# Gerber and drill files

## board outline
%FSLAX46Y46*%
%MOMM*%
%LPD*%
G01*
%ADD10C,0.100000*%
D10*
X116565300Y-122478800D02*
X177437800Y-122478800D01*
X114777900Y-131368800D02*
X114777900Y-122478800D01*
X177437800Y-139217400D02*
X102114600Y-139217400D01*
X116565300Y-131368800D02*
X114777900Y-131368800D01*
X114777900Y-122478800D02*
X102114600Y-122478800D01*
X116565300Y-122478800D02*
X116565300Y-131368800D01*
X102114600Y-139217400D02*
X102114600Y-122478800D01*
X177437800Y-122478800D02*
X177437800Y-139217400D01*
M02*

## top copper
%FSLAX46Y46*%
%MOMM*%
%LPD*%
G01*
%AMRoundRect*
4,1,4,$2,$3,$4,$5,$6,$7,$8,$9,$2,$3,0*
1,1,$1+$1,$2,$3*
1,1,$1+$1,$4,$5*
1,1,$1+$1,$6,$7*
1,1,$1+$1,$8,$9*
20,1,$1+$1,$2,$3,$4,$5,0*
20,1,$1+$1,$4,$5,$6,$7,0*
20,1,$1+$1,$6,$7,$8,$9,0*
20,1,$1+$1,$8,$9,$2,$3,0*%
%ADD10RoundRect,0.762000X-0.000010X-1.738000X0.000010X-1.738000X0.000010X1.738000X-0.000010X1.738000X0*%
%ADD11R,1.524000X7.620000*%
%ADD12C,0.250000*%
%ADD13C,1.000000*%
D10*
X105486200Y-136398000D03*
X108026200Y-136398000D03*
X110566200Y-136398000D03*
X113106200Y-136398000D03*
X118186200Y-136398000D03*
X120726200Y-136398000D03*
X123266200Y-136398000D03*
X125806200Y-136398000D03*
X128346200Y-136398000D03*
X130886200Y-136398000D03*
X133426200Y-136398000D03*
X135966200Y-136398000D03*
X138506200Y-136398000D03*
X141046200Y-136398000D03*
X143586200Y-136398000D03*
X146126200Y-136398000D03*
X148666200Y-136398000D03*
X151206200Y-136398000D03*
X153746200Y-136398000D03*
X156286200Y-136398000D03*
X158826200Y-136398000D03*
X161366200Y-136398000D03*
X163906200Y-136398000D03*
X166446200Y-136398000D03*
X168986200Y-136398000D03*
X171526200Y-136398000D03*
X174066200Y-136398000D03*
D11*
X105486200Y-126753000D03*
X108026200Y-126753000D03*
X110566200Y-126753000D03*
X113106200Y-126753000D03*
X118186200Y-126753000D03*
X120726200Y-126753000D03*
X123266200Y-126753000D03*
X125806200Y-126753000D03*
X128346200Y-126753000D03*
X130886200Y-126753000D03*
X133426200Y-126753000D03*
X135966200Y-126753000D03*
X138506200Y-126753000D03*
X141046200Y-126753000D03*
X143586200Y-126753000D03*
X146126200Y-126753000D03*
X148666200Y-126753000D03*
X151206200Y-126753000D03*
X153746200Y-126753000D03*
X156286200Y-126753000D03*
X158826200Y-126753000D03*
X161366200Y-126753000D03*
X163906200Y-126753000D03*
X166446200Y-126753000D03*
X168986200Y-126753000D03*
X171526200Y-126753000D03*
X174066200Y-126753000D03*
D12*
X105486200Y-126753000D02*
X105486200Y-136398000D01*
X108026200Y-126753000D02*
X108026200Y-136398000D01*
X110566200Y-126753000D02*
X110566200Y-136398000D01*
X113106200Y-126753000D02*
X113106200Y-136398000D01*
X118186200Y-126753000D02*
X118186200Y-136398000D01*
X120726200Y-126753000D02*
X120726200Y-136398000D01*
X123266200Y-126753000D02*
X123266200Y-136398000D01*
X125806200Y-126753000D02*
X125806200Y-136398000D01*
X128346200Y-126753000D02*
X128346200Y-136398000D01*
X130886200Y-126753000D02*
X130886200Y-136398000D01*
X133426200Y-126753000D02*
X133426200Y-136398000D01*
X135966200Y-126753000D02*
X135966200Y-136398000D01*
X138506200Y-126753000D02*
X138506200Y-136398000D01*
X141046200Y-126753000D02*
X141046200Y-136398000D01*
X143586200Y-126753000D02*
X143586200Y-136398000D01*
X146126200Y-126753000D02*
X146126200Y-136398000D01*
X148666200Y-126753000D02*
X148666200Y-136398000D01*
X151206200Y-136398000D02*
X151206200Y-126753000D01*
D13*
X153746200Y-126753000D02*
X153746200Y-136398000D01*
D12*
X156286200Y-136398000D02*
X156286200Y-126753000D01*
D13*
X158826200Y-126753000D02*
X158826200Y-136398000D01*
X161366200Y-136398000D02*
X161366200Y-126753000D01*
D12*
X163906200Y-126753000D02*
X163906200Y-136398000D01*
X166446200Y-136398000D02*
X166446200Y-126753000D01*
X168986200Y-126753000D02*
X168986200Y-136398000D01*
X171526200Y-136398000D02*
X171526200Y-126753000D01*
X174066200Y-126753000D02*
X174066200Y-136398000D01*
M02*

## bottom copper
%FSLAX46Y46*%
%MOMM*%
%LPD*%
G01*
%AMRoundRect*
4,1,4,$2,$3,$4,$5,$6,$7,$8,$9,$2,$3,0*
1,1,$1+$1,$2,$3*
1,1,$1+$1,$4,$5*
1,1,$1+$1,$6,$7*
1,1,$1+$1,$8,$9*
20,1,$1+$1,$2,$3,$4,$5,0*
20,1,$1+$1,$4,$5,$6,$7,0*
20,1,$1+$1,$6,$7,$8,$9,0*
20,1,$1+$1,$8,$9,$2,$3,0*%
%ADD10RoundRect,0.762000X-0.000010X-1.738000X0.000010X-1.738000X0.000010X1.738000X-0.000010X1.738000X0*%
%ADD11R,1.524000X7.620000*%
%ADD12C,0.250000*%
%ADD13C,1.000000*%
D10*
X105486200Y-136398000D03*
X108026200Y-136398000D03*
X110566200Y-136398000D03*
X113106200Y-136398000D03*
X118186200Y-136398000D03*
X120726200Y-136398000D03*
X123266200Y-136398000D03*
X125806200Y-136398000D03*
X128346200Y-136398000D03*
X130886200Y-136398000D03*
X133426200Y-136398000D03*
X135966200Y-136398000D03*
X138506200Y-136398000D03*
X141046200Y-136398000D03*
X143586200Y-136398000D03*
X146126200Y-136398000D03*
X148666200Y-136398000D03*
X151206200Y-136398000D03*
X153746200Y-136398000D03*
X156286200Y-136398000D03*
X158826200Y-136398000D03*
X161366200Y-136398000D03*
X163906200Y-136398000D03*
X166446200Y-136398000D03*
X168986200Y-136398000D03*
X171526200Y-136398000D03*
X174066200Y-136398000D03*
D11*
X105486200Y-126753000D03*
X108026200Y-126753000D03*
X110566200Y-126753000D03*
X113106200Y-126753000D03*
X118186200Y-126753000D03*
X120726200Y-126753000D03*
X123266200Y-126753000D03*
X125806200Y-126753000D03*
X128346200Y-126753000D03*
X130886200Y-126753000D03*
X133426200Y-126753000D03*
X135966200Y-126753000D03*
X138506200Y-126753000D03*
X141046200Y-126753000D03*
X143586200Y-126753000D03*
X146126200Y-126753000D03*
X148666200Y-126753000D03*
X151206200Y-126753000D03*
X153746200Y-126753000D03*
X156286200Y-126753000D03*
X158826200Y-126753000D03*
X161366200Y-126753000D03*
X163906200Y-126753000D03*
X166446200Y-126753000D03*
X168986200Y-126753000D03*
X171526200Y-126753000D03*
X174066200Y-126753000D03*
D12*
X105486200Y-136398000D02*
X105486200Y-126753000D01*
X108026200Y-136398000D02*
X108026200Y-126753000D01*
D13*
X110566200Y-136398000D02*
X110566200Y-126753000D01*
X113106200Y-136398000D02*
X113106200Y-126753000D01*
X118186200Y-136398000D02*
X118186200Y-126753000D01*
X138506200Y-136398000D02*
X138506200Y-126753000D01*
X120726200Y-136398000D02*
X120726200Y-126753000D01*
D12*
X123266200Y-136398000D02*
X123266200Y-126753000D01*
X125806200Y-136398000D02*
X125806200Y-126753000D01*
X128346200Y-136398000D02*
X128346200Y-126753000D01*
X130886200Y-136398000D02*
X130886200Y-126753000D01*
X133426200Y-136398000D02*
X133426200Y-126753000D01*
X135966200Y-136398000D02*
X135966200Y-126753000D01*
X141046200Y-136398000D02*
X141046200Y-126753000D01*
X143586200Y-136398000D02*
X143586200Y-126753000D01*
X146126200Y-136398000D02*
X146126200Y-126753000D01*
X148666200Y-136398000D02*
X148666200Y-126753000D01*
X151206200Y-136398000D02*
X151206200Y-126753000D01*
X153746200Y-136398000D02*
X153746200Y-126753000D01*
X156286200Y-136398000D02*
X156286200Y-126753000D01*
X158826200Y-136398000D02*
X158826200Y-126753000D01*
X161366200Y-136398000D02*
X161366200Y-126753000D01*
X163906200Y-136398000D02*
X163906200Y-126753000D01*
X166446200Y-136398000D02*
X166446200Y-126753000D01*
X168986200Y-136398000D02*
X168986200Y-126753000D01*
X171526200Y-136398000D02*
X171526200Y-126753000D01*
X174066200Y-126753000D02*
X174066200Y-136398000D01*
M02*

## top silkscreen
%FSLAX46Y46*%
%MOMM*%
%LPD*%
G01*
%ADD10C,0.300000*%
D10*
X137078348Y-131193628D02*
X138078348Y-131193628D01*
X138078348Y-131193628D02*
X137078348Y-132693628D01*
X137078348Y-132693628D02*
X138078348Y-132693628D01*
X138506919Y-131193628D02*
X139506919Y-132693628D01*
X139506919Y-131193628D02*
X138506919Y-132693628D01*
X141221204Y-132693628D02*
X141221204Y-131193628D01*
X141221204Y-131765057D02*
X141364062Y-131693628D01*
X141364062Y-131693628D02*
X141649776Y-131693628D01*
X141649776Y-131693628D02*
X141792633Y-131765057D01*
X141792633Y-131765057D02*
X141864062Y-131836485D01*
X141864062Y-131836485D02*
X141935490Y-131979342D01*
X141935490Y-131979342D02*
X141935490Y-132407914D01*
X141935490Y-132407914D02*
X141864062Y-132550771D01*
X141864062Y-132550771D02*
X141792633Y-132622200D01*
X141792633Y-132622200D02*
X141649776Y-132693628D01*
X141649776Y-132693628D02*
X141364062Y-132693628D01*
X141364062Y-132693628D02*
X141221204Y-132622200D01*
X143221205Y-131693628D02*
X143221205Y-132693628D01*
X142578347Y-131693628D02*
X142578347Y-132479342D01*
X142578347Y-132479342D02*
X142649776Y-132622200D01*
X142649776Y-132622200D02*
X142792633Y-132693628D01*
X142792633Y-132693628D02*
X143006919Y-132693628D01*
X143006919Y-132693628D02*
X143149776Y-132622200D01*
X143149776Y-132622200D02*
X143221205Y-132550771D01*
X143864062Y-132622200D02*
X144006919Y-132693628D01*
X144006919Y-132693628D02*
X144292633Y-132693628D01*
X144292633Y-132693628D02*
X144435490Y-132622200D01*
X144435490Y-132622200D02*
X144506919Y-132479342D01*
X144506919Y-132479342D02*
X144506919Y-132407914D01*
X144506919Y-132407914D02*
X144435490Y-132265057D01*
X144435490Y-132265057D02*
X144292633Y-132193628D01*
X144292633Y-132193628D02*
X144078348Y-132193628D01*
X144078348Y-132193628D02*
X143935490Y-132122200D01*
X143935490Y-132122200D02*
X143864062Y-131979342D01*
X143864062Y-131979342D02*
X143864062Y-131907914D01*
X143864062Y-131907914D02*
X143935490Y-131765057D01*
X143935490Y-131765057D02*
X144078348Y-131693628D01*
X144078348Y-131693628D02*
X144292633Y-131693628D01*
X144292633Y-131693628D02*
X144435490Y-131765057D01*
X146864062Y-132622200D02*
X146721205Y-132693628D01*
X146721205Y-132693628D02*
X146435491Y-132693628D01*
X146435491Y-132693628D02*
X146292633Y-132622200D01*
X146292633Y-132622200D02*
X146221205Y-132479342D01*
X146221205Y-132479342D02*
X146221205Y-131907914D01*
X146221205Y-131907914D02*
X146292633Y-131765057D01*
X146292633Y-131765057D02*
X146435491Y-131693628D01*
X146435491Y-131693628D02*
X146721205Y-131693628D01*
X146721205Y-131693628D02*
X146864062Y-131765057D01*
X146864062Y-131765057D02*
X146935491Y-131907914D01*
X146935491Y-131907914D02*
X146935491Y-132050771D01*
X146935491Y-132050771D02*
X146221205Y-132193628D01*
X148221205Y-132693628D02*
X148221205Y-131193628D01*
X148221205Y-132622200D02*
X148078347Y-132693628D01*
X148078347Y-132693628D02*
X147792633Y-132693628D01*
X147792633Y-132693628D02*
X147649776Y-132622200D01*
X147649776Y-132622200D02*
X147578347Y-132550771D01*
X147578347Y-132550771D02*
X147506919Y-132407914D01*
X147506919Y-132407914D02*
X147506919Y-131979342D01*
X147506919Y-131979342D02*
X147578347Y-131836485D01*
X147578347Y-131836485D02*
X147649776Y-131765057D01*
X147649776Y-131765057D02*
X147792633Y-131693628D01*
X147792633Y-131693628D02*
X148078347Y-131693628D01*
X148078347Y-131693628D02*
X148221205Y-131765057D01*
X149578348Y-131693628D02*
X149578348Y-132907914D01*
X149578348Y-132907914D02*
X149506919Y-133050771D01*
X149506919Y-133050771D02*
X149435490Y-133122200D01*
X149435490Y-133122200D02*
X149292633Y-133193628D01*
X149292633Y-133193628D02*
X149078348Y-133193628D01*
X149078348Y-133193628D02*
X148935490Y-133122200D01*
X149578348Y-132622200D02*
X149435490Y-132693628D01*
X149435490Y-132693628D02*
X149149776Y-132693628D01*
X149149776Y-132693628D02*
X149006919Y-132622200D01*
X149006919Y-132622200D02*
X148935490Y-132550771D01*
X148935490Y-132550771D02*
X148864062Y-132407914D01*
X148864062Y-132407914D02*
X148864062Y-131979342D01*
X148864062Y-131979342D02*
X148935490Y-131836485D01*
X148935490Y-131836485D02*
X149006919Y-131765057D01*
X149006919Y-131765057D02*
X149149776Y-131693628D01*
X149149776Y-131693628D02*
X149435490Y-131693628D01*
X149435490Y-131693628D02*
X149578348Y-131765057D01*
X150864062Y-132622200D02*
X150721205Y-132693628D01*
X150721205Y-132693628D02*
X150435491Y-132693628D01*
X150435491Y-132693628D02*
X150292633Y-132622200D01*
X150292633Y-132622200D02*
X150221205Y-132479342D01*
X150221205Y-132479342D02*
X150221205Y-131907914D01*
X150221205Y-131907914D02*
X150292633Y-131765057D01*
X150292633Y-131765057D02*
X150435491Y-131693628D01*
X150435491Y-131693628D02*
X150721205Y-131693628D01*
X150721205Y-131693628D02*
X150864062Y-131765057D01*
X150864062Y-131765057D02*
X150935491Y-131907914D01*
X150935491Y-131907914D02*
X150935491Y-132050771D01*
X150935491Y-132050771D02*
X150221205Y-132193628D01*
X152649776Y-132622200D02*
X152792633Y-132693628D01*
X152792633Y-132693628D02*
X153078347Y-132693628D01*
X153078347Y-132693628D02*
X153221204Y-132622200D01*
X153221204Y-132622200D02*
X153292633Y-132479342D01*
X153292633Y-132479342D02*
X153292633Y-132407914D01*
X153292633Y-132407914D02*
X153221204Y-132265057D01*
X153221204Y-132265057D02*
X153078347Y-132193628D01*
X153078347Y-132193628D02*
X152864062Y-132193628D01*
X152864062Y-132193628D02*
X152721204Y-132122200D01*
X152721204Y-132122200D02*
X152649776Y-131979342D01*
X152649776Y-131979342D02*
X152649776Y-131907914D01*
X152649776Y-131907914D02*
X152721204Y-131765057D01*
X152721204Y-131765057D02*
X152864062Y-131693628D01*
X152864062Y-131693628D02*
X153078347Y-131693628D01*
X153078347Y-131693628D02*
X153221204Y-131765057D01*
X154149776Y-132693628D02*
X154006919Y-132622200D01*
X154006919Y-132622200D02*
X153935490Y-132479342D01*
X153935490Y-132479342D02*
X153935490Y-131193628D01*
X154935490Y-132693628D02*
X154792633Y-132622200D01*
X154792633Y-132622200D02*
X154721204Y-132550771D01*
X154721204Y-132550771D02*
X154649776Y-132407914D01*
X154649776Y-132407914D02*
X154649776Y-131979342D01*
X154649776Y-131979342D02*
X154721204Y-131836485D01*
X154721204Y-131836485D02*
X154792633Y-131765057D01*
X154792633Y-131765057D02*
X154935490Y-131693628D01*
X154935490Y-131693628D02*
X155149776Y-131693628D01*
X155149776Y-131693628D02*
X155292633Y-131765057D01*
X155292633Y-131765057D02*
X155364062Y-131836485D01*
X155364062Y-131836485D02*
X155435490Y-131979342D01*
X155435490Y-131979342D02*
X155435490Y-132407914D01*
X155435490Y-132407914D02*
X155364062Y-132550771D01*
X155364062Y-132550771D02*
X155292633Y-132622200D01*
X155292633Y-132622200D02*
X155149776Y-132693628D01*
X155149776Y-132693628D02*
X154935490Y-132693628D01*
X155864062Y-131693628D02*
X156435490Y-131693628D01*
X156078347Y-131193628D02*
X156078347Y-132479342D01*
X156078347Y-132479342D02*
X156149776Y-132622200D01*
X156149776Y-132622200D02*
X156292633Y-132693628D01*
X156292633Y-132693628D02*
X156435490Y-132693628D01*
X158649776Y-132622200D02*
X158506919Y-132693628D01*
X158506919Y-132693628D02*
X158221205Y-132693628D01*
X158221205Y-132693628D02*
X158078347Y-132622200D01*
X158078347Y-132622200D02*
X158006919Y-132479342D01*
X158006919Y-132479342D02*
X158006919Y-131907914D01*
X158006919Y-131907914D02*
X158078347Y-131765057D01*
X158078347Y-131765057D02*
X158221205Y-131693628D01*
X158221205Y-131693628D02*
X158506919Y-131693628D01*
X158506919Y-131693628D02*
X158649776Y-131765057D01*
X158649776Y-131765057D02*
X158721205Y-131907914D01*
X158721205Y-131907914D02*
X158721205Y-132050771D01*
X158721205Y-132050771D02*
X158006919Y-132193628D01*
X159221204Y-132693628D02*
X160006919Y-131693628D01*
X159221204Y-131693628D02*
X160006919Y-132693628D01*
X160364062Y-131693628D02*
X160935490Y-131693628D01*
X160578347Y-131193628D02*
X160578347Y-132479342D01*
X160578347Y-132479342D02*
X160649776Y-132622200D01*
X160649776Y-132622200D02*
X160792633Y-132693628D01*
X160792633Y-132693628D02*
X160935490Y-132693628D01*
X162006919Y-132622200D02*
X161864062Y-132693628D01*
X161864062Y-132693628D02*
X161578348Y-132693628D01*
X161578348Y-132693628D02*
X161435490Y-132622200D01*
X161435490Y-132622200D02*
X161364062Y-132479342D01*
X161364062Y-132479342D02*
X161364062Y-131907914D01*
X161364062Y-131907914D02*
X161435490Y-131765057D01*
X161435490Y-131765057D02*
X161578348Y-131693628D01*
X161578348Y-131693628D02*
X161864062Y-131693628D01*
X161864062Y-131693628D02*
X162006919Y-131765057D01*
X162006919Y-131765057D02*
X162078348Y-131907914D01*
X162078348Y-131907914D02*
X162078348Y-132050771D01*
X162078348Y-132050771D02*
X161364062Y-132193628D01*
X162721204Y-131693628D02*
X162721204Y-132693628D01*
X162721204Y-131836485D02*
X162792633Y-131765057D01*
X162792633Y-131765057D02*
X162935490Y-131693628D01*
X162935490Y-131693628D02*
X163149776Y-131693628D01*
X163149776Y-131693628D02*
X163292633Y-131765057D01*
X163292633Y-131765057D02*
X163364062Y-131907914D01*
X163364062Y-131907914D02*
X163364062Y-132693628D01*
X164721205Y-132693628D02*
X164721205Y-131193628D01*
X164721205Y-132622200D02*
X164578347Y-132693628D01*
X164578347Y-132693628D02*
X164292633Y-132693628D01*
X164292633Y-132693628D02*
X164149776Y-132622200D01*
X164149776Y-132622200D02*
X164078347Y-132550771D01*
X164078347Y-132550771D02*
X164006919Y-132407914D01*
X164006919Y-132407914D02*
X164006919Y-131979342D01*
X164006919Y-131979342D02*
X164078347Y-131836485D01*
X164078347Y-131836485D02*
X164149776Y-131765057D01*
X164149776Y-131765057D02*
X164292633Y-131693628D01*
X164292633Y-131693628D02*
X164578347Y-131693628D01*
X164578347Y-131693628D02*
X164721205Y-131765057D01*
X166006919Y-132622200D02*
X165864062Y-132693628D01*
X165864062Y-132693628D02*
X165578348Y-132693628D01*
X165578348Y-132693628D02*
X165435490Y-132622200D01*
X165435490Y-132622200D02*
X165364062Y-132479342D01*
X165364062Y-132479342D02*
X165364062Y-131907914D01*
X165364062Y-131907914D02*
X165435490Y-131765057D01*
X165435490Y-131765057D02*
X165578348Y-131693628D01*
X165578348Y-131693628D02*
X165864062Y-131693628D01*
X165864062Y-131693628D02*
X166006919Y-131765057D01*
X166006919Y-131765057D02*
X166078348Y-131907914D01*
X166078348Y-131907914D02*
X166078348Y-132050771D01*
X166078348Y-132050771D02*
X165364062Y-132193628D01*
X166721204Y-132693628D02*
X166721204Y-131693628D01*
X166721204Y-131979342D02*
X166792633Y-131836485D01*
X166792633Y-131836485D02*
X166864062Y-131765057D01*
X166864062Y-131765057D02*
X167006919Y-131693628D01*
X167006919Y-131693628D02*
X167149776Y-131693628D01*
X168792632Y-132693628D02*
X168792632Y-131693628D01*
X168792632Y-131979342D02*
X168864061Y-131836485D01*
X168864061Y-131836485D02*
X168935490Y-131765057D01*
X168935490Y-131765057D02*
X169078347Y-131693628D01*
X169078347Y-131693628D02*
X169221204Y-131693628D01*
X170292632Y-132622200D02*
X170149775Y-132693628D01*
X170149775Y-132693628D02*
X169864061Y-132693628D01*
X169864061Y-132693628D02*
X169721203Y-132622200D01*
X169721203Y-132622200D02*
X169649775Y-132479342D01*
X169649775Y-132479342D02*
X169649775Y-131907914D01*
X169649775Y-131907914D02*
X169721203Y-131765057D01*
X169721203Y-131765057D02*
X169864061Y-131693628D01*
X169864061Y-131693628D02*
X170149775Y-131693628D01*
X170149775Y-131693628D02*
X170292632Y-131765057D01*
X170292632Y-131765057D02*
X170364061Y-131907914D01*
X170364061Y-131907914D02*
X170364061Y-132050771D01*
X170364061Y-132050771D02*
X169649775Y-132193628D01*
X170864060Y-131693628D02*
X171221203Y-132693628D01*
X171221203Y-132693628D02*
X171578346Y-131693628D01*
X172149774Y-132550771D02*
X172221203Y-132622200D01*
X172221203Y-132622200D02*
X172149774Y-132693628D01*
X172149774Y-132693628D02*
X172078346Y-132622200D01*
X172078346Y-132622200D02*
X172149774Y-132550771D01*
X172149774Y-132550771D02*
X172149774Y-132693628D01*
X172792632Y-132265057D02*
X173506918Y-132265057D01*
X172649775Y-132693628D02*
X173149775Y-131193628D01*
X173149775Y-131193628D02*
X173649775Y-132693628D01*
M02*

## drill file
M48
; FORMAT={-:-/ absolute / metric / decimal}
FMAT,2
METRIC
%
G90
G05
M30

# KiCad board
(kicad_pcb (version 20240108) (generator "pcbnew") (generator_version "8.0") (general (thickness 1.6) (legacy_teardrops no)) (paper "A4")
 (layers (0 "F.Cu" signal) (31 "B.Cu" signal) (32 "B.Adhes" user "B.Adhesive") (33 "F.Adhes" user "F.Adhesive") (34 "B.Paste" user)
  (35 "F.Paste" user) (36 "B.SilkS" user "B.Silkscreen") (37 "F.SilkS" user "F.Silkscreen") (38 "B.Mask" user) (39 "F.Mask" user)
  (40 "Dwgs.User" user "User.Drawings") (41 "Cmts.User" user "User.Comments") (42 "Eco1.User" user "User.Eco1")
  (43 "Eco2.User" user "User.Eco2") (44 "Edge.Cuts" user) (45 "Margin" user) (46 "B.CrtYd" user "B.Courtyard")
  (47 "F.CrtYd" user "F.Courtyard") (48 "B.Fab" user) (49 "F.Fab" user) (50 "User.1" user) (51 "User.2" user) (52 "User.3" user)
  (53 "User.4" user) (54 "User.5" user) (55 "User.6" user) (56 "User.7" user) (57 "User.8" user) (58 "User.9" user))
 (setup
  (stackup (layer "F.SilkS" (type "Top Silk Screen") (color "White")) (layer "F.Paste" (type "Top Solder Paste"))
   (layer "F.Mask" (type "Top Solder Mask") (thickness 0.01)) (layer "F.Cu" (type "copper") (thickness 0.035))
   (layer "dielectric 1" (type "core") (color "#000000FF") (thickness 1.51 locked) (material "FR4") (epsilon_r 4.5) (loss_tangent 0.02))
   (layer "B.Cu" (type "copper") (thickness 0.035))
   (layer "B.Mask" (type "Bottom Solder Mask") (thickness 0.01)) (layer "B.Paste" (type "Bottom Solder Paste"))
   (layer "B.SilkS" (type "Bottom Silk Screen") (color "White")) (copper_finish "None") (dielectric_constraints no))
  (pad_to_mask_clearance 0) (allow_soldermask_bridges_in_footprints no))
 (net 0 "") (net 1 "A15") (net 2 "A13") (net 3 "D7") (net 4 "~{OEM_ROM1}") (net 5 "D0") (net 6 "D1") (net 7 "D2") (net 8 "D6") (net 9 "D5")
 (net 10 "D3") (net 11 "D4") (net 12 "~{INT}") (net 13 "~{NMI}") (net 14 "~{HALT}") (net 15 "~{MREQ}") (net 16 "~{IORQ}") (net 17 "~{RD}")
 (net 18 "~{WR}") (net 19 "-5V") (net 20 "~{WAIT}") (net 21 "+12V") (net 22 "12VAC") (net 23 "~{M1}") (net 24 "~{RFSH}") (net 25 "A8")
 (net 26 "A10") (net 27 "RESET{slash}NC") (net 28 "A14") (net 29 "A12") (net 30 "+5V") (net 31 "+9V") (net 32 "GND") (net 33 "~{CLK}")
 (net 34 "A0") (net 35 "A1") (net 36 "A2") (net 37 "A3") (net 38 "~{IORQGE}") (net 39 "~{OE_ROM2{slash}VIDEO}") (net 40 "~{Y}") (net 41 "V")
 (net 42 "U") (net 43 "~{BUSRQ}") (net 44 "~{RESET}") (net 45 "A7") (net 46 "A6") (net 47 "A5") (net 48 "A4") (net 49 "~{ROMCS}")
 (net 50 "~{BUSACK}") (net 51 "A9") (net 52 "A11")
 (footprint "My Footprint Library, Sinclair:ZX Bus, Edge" (layer "F.Cu") (at 138.5062 136.398)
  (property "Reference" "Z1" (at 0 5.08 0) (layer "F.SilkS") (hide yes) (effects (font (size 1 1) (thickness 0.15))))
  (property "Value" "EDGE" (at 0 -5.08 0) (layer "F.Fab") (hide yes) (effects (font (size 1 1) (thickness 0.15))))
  (pad "A1" smd roundrect (at -33.02 0) (size 1.524 5) (layers "F.Cu" "F.Paste" "F.Mask") (roundrect_rratio 0.5) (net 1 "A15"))
  (pad "A2" smd roundrect (at -30.48 0) (size 1.524 5) (layers "F.Cu" "F.Paste" "F.Mask") (roundrect_rratio 0.5) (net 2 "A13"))
  (pad "A3" smd roundrect (at -27.94 0) (size 1.524 5) (layers "F.Cu" "F.Paste" "F.Mask") (roundrect_rratio 0.5) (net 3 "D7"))
  (pad "A4" smd roundrect (at -25.4 0) (size 1.524 5) (layers "F.Cu" "F.Paste" "F.Mask") (roundrect_rratio 0.5) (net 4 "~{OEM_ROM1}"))
  (pad "A6" smd roundrect (at -20.32 0) (size 1.524 5) (layers "F.Cu" "F.Paste" "F.Mask") (roundrect_rratio 0.5) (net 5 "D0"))
  (pad "A7" smd roundrect (at -17.78 0) (size 1.524 5) (layers "F.Cu" "F.Paste" "F.Mask") (roundrect_rratio 0.5) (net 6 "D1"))
  (pad "A8" smd roundrect (at -15.24 0) (size 1.524 5) (layers "F.Cu" "F.Paste" "F.Mask") (roundrect_rratio 0.5) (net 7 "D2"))
  (pad "A9" smd roundrect (at -12.7 0) (size 1.524 5) (layers "F.Cu" "F.Paste" "F.Mask") (roundrect_rratio 0.5) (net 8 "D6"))
  (pad "A10" smd roundrect (at -10.16 0) (size 1.524 5) (layers "F.Cu" "F.Paste" "F.Mask") (roundrect_rratio 0.5) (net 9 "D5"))
  (pad "A11" smd roundrect (at -7.62 0) (size 1.524 5) (layers "F.Cu" "F.Paste" "F.Mask") (roundrect_rratio 0.5) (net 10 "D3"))
  (pad "A12" smd roundrect (at -5.08 0) (size 1.524 5) (layers "F.Cu" "F.Paste" "F.Mask") (roundrect_rratio 0.5) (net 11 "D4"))
  (pad "A13" smd roundrect (at -2.54 0) (size 1.524 5) (layers "F.Cu" "F.Paste" "F.Mask") (roundrect_rratio 0.5) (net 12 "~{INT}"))
  (pad "A14" smd roundrect (at 0 0) (size 1.524 5) (layers "F.Cu" "F.Paste" "F.Mask") (roundrect_rratio 0.5) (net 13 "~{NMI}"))
  (pad "A15" smd roundrect (at 2.54 0) (size 1.524 5) (layers "F.Cu" "F.Paste" "F.Mask") (roundrect_rratio 0.5) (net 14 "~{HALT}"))
  (pad "A16" smd roundrect (at 5.08 0) (size 1.524 5) (layers "F.Cu" "F.Paste" "F.Mask") (roundrect_rratio 0.5) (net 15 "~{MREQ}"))
  (pad "A17" smd roundrect (at 7.62 0) (size 1.524 5) (layers "F.Cu" "F.Paste" "F.Mask") (roundrect_rratio 0.5) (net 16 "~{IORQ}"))
  (pad "A18" smd roundrect (at 10.16 0) (size 1.524 5) (layers "F.Cu" "F.Paste" "F.Mask") (roundrect_rratio 0.5) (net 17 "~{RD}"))
  (pad "A19" smd roundrect (at 12.7 0) (size 1.524 5) (layers "F.Cu" "F.Paste" "F.Mask") (roundrect_rratio 0.5) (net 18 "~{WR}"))
  (pad "A20" smd roundrect (at 15.24 0) (size 1.524 5) (layers "F.Cu" "F.Paste" "F.Mask") (roundrect_rratio 0.5) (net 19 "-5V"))
  (pad "A21" smd roundrect (at 17.78 0) (size 1.524 5) (layers "F.Cu" "F.Paste" "F.Mask") (roundrect_rratio 0.5) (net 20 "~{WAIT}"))
  (pad "A22" smd roundrect (at 20.32 0) (size 1.524 5) (layers "F.Cu" "F.Paste" "F.Mask") (roundrect_rratio 0.5) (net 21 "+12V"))
  (pad "A23" smd roundrect (at 22.86 0) (size 1.524 5) (layers "F.Cu" "F.Paste" "F.Mask") (roundrect_rratio 0.5) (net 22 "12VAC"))
  (pad "A24" smd roundrect (at 25.4 0) (size 1.524 5) (layers "F.Cu" "F.Paste" "F.Mask") (roundrect_rratio 0.5) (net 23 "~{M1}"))
  (pad "A25" smd roundrect (at 27.94 0) (size 1.524 5) (layers "F.Cu" "F.Paste" "F.Mask") (roundrect_rratio 0.5) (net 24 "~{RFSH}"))
  (pad "A26" smd roundrect (at 30.48 0) (size 1.524 5) (layers "F.Cu" "F.Paste" "F.Mask") (roundrect_rratio 0.5) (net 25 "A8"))
  (pad "A27" smd roundrect (at 33.02 0) (size 1.524 5) (layers "F.Cu" "F.Paste" "F.Mask") (roundrect_rratio 0.5) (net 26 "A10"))
  (pad "A28" smd roundrect (at 35.56 0) (size 1.524 5) (layers "F.Cu" "F.Paste" "F.Mask") (roundrect_rratio 0.5) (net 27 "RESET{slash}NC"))
  (pad "B1" smd roundrect (at -33.02 0) (size 1.524 5) (layers "B.Cu" "B.Paste" "B.Mask") (roundrect_rratio 0.5) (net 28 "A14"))
  (pad "B2" smd roundrect (at -30.48 0) (size 1.524 5) (layers "B.Cu" "B.Paste" "B.Mask") (roundrect_rratio 0.5) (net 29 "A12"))
  (pad "B3" smd roundrect (at -27.94 0) (size 1.524 5) (layers "B.Cu" "B.Paste" "B.Mask") (roundrect_rratio 0.5) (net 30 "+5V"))
  (pad "B4" smd roundrect (at -25.4 0) (size 1.524 5) (layers "B.Cu" "B.Paste" "B.Mask") (roundrect_rratio 0.5) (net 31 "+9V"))
  (pad "B6" smd roundrect (at -20.32 0) (size 1.524 5) (layers "B.Cu" "B.Paste" "B.Mask") (roundrect_rratio 0.5) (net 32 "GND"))
  (pad "B7" smd roundrect (at -17.78 0) (size 1.524 5) (layers "B.Cu" "B.Paste" "B.Mask") (roundrect_rratio 0.5) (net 32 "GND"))
  (pad "B8" smd roundrect (at -15.24 0) (size 1.524 5) (layers "B.Cu" "B.Paste" "B.Mask") (roundrect_rratio 0.5) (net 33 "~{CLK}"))
  (pad "B9" smd roundrect (at -12.7 0) (size 1.524 5) (layers "B.Cu" "B.Paste" "B.Mask") (roundrect_rratio 0.5) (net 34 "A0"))
  (pad "B10" smd roundrect (at -10.16 0) (size 1.524 5) (layers "B.Cu" "B.Paste" "B.Mask") (roundrect_rratio 0.5) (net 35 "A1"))
  (pad "B11" smd roundrect (at -7.62 0) (size 1.524 5) (layers "B.Cu" "B.Paste" "B.Mask") (roundrect_rratio 0.5) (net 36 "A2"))
  (pad "B12" smd roundrect (at -5.08 0) (size 1.524 5) (layers "B.Cu" "B.Paste" "B.Mask") (roundrect_rratio 0.5) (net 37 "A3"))
  (pad "B13" smd roundrect (at -2.54 0) (size 1.524 5) (layers "B.Cu" "B.Paste" "B.Mask") (roundrect_rratio 0.5) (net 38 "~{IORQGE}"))
  (pad "B14" smd roundrect (at 0 0) (size 1.524 5) (layers "B.Cu" "B.Paste" "B.Mask") (roundrect_rratio 0.5) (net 32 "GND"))
  (pad "B15" smd roundrect (at 2.54 0) (size 1.524 5) (layers "B.Cu" "B.Paste" "B.Mask") (roundrect_rratio 0.5)
   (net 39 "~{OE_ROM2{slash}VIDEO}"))
  (pad "B16" smd roundrect (at 5.08 0) (size 1.524 5) (layers "B.Cu" "B.Paste" "B.Mask") (roundrect_rratio 0.5) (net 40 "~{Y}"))
  (pad "B17" smd roundrect (at 7.62 0) (size 1.524 5) (layers "B.Cu" "B.Paste" "B.Mask") (roundrect_rratio 0.5) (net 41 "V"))
  (pad "B18" smd roundrect (at 10.16 0) (size 1.524 5) (layers "B.Cu" "B.Paste" "B.Mask") (roundrect_rratio 0.5) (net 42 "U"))
  (pad "B19" smd roundrect (at 12.7 0) (size 1.524 5) (layers "B.Cu" "B.Paste" "B.Mask") (roundrect_rratio 0.5) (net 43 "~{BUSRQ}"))
  (pad "B20" smd roundrect (at 15.24 0) (size 1.524 5) (layers "B.Cu" "B.Paste" "B.Mask") (roundrect_rratio 0.5) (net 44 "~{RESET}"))
  (pad "B21" smd roundrect (at 17.78 0) (size 1.524 5) (layers "B.Cu" "B.Paste" "B.Mask") (roundrect_rratio 0.5) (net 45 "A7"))
  (pad "B22" smd roundrect (at 20.32 0) (size 1.524 5) (layers "B.Cu" "B.Paste" "B.Mask") (roundrect_rratio 0.5) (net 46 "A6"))
  (pad "B23" smd roundrect (at 22.86 0) (size 1.524 5) (layers "B.Cu" "B.Paste" "B.Mask") (roundrect_rratio 0.5) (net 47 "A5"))
  (pad "B24" smd roundrect (at 25.4 0) (size 1.524 5) (layers "B.Cu" "B.Paste" "B.Mask") (roundrect_rratio 0.5) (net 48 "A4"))
  (pad "B25" smd roundrect (at 27.94 0) (size 1.524 5) (layers "B.Cu" "B.Paste" "B.Mask") (roundrect_rratio 0.5) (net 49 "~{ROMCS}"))
  (pad "B26" smd roundrect (at 30.48 0) (size 1.524 5) (layers "B.Cu" "B.Paste" "B.Mask") (roundrect_rratio 0.5) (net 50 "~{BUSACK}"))
  (pad "B27" smd roundrect (at 33.02 0) (size 1.524 5) (layers "B.Cu" "B.Paste" "B.Mask") (roundrect_rratio 0.5) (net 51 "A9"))
  (pad "B28" smd roundrect (at 35.56 0) (size 1.524 5) (layers "B.Cu" "B.Paste" "B.Mask") (roundrect_rratio 0.5) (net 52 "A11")))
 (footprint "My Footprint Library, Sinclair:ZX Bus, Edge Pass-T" (layer "F.Cu") (at 138.5062 126.753)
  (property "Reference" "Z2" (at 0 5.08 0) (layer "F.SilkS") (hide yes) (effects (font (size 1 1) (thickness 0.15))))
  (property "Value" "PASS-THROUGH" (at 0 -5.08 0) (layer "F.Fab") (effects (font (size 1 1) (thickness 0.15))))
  (pad "A1" smd rect (at -33.02 0) (size 1.524 7.62) (layers "F.Cu" "F.Paste" "F.Mask") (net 1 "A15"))
  (pad "A2" smd rect (at -30.48 0) (size 1.524 7.62) (layers "F.Cu" "F.Paste" "F.Mask") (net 2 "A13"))
  (pad "A3" smd rect (at -27.94 0) (size 1.524 7.62) (layers "F.Cu" "F.Paste" "F.Mask") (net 3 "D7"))
  (pad "A4" smd rect (at -25.4 0) (size 1.524 7.62) (layers "F.Cu" "F.Paste" "F.Mask") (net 4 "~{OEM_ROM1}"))
  (pad "A6" smd rect (at -20.32 0) (size 1.524 7.62) (layers "F.Cu" "F.Paste" "F.Mask") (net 5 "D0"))
  (pad "A7" smd rect (at -17.78 0) (size 1.524 7.62) (layers "F.Cu" "F.Paste" "F.Mask") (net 6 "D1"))
  (pad "A8" smd rect (at -15.24 0) (size 1.524 7.62) (layers "F.Cu" "F.Paste" "F.Mask") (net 7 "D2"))
  (pad "A9" smd rect (at -12.7 0) (size 1.524 7.62) (layers "F.Cu" "F.Paste" "F.Mask") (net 8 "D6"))
  (pad "A10" smd rect (at -10.16 0) (size 1.524 7.62) (layers "F.Cu" "F.Paste" "F.Mask") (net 9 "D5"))
  (pad "A11" smd rect (at -7.62 0) (size 1.524 7.62) (layers "F.Cu" "F.Paste" "F.Mask") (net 10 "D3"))
  (pad "A12" smd rect (at -5.08 0) (size 1.524 7.62) (layers "F.Cu" "F.Paste" "F.Mask") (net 11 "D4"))
  (pad "A13" smd rect (at -2.54 0) (size 1.524 7.62) (layers "F.Cu" "F.Paste" "F.Mask") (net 12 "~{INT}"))
  (pad "A14" smd rect (at 0 0) (size 1.524 7.62) (layers "F.Cu" "F.Paste" "F.Mask") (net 13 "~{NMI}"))
  (pad "A15" smd rect (at 2.54 0) (size 1.524 7.62) (layers "F.Cu" "F.Paste" "F.Mask") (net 14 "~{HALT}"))
  (pad "A16" smd rect (at 5.08 0) (size 1.524 7.62) (layers "F.Cu" "F.Paste" "F.Mask") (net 15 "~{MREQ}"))
  (pad "A17" smd rect (at 7.62 0) (size 1.524 7.62) (layers "F.Cu" "F.Paste" "F.Mask") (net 16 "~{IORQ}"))
  (pad "A18" smd rect (at 10.16 0) (size 1.524 7.62) (layers "F.Cu" "F.Paste" "F.Mask") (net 17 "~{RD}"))
  (pad "A19" smd rect (at 12.7 0) (size 1.524 7.62) (layers "F.Cu" "F.Paste" "F.Mask") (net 18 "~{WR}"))
  (pad "A20" smd rect (at 15.24 0) (size 1.524 7.62) (layers "F.Cu" "F.Paste" "F.Mask") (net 19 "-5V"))
  (pad "A21" smd rect (at 17.78 0) (size 1.524 7.62) (layers "F.Cu" "F.Paste" "F.Mask") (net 20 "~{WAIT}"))
  (pad "A22" smd rect (at 20.32 0) (size 1.524 7.62) (layers "F.Cu" "F.Paste" "F.Mask") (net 21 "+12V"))
  (pad "A23" smd rect (at 22.86 0) (size 1.524 7.62) (layers "F.Cu" "F.Paste" "F.Mask") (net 22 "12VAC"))
  (pad "A24" smd rect (at 25.4 0) (size 1.524 7.62) (layers "F.Cu" "F.Paste" "F.Mask") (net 23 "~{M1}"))
  (pad "A25" smd rect (at 27.94 0) (size 1.524 7.62) (layers "F.Cu" "F.Paste" "F.Mask") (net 24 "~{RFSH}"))
  (pad "A26" smd rect (at 30.48 0) (size 1.524 7.62) (layers "F.Cu" "F.Paste" "F.Mask") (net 25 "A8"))
  (pad "A27" smd rect (at 33.02 0) (size 1.524 7.62) (layers "F.Cu" "F.Paste" "F.Mask") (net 26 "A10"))
  (pad "A28" smd rect (at 35.56 0) (size 1.524 7.62) (layers "F.Cu" "F.Paste" "F.Mask") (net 27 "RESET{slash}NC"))
  (pad "B1" smd rect (at -33.02 0) (size 1.524 7.62) (layers "B.Cu" "B.Paste" "B.Mask") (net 28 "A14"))
  (pad "B2" smd rect (at -30.48 0) (size 1.524 7.62) (layers "B.Cu" "B.Paste" "B.Mask") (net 29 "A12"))
  (pad "B3" smd rect (at -27.94 0) (size 1.524 7.62) (layers "B.Cu" "B.Paste" "B.Mask") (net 30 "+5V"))
  (pad "B4" smd rect (at -25.4 0) (size 1.524 7.62) (layers "B.Cu" "B.Paste" "B.Mask") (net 31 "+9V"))
  (pad "B6" smd rect (at -20.32 0) (size 1.524 7.62) (layers "B.Cu" "B.Paste" "B.Mask") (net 32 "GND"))
  (pad "B7" smd rect (at -17.78 0) (size 1.524 7.62) (layers "B.Cu" "B.Paste" "B.Mask") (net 32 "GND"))
  (pad "B8" smd rect (at -15.24 0) (size 1.524 7.62) (layers "B.Cu" "B.Paste" "B.Mask") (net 33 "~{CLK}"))
  (pad "B9" smd rect (at -12.7 0) (size 1.524 7.62) (layers "B.Cu" "B.Paste" "B.Mask") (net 34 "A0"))
  (pad "B10" smd rect (at -10.16 0) (size 1.524 7.62) (layers "B.Cu" "B.Paste" "B.Mask") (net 35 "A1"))
  (pad "B11" smd rect (at -7.62 0) (size 1.524 7.62) (layers "B.Cu" "B.Paste" "B.Mask") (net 36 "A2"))
  (pad "B12" smd rect (at -5.08 0) (size 1.524 7.62) (layers "B.Cu" "B.Paste" "B.Mask") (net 37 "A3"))
  (pad "B13" smd rect (at -2.54 0) (size 1.524 7.62) (layers "B.Cu" "B.Paste" "B.Mask") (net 38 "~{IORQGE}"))
  (pad "B14" smd rect (at 0 0) (size 1.524 7.62) (layers "B.Cu" "B.Paste" "B.Mask") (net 32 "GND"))
  (pad "B15" smd rect (at 2.54 0) (size 1.524 7.62) (layers "B.Cu" "B.Paste" "B.Mask") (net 39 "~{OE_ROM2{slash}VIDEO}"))
  (pad "B16" smd rect (at 5.08 0) (size 1.524 7.62) (layers "B.Cu" "B.Paste" "B.Mask") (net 40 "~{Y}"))
  (pad "B17" smd rect (at 7.62 0) (size 1.524 7.62) (layers "B.Cu" "B.Paste" "B.Mask") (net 41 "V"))
  (pad "B18" smd rect (at 10.16 0) (size 1.524 7.62) (layers "B.Cu" "B.Paste" "B.Mask") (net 42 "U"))
  (pad "B19" smd rect (at 12.7 0) (size 1.524 7.62) (layers "B.Cu" "B.Paste" "B.Mask") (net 43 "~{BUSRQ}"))
  (pad "B20" smd rect (at 15.24 0) (size 1.524 7.62) (layers "B.Cu" "B.Paste" "B.Mask") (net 44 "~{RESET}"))
  (pad "B21" smd rect (at 17.78 0) (size 1.524 7.62) (layers "B.Cu" "B.Paste" "B.Mask") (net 45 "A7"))
  (pad "B22" smd rect (at 20.32 0) (size 1.524 7.62) (layers "B.Cu" "B.Paste" "B.Mask") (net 46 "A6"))
  (pad "B23" smd rect (at 22.86 0) (size 1.524 7.62) (layers "B.Cu" "B.Paste" "B.Mask") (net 47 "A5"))
  (pad "B24" smd rect (at 25.4 0) (size 1.524 7.62) (layers "B.Cu" "B.Paste" "B.Mask") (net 48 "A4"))
  (pad "B25" smd rect (at 27.94 0) (size 1.524 7.62) (layers "B.Cu" "B.Paste" "B.Mask") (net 49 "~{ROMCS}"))
  (pad "B26" smd rect (at 30.48 0) (size 1.524 7.62) (layers "B.Cu" "B.Paste" "B.Mask") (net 50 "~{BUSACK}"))
  (pad "B27" smd rect (at 33.02 0) (size 1.524 7.62) (layers "B.Cu" "B.Paste" "B.Mask") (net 51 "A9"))
  (pad "B28" smd rect (at 35.56 0) (size 1.524 7.62) (layers "B.Cu" "B.Paste" "B.Mask") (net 52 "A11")))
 (gr_line (start 116.5653 122.4788) (end 177.4378 122.4788) (stroke (width 0.1) (type default)) (layer "Edge.Cuts"))
 (gr_line (start 114.7779 131.3688) (end 114.7779 122.4788) (stroke (width 0.1) (type default)) (layer "Edge.Cuts"))
 (gr_line (start 177.4378 139.2174) (end 102.1146 139.2174) (stroke (width 0.1) (type default)) (layer "Edge.Cuts"))
 (gr_line (start 116.5653 131.3688) (end 114.7779 131.3688) (stroke (width 0.1) (type default)) (layer "Edge.Cuts"))
 (gr_line (start 114.7779 122.4788) (end 102.1146 122.4788) (stroke (width 0.1) (type default)) (layer "Edge.Cuts"))
 (gr_line (start 116.5653 122.4788) (end 116.5653 131.3688) (stroke (width 0.1) (type default)) (layer "Edge.Cuts"))
 (gr_line (start 102.1146 139.2174) (end 102.1146 122.4788) (stroke (width 0.1) (type default)) (layer "Edge.Cuts"))
 (gr_line (start 177.4378 122.4788) (end 177.4378 139.2174) (stroke (width 0.1) (type default)) (layer "Edge.Cuts"))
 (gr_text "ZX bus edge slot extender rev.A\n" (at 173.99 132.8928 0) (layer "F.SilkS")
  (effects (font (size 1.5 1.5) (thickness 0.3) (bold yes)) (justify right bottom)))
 (segment (start 105.4862 126.753) (end 105.4862 136.398) (width 0.25) (layer "F.Cu") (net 1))
 (segment (start 108.0262 126.753) (end 108.0262 136.398) (width 0.25) (layer "F.Cu") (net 2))
 (segment (start 110.5662 126.753) (end 110.5662 136.398) (width 0.25) (layer "F.Cu") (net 3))
 (segment (start 113.1062 126.753) (end 113.1062 136.398) (width 0.25) (layer "F.Cu") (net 4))
 (segment (start 118.1862 126.753) (end 118.1862 136.398) (width 0.25) (layer "F.Cu") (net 5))
 (segment (start 120.7262 126.753) (end 120.7262 136.398) (width 0.25) (layer "F.Cu") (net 6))
 (segment (start 123.2662 126.753) (end 123.2662 136.398) (width 0.25) (layer "F.Cu") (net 7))
 (segment (start 125.8062 126.753) (end 125.8062 136.398) (width 0.25) (layer "F.Cu") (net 8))
 (segment (start 128.3462 126.753) (end 128.3462 136.398) (width 0.25) (layer "F.Cu") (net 9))
 (segment (start 130.8862 126.753) (end 130.8862 136.398) (width 0.25) (layer "F.Cu") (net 10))
 (segment (start 133.4262 126.753) (end 133.4262 136.398) (width 0.25) (layer "F.Cu") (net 11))
 (segment (start 135.9662 126.753) (end 135.9662 136.398) (width 0.25) (layer "F.Cu") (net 12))
 (segment (start 138.5062 126.753) (end 138.5062 136.398) (width 0.25) (layer "F.Cu") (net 13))
 (segment (start 141.0462 126.753) (end 141.0462 136.398) (width 0.25) (layer "F.Cu") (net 14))
 (segment (start 143.5862 126.753) (end 143.5862 136.398) (width 0.25) (layer "F.Cu") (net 15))
 (segment (start 146.1262 126.753) (end 146.1262 136.398) (width 0.25) (layer "F.Cu") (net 16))
 (segment (start 148.6662 126.753) (end 148.6662 136.398) (width 0.25) (layer "F.Cu") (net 17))
 (segment (start 151.2062 136.398) (end 151.2062 126.753) (width 0.25) (layer "F.Cu") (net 18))
 (segment (start 153.7462 126.753) (end 153.7462 136.398) (width 1) (layer "F.Cu") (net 19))
 (segment (start 156.2862 136.398) (end 156.2862 126.753) (width 0.25) (layer "F.Cu") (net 20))
 (segment (start 158.8262 126.753) (end 158.8262 136.398) (width 1) (layer "F.Cu") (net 21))
 (segment (start 161.3662 136.398) (end 161.3662 126.753) (width 1) (layer "F.Cu") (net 22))
 (segment (start 163.9062 126.753) (end 163.9062 136.398) (width 0.25) (layer "F.Cu") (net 23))
 (segment (start 166.4462 136.398) (end 166.4462 126.753) (width 0.25) (layer "F.Cu") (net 24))
 (segment (start 168.9862 126.753) (end 168.9862 136.398) (width 0.25) (layer "F.Cu") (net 25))
 (segment (start 171.5262 136.398) (end 171.5262 126.753) (width 0.25) (layer "F.Cu") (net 26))
 (segment (start 174.0662 126.753) (end 174.0662 136.398) (width 0.25) (layer "F.Cu") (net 27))
 (segment (start 105.4862 136.398) (end 105.4862 126.753) (width 0.25) (layer "B.Cu") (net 28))
 (segment (start 108.0262 136.398) (end 108.0262 126.753) (width 0.25) (layer "B.Cu") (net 29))
 (segment (start 110.5662 136.398) (end 110.5662 126.753) (width 1) (layer "B.Cu") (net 30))
 (segment (start 113.1062 136.398) (end 113.1062 126.753) (width 1) (layer "B.Cu") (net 31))
 (segment (start 118.1862 136.398) (end 118.1862 126.753) (width 1) (layer "B.Cu") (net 32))
 (segment (start 138.5062 136.398) (end 138.5062 126.753) (width 1) (layer "B.Cu") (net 32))
 (segment (start 120.7262 136.398) (end 120.7262 126.753) (width 1) (layer "B.Cu") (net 32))
 (segment (start 123.2662 136.398) (end 123.2662 126.753) (width 0.25) (layer "B.Cu") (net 33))
 (segment (start 125.8062 136.398) (end 125.8062 126.753) (width 0.25) (layer "B.Cu") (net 34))
 (segment (start 128.3462 136.398) (end 128.3462 126.753) (width 0.25) (layer "B.Cu") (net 35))
 (segment (start 130.8862 136.398) (end 130.8862 126.753) (width 0.25) (layer "B.Cu") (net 36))
 (segment (start 133.4262 136.398) (end 133.4262 126.753) (width 0.25) (layer "B.Cu") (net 37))
 (segment (start 135.9662 136.398) (end 135.9662 126.753) (width 0.25) (layer "B.Cu") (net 38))
 (segment (start 141.0462 136.398) (end 141.0462 126.753) (width 0.25) (layer "B.Cu") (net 39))
 (segment (start 143.5862 136.398) (end 143.5862 126.753) (width 0.25) (layer "B.Cu") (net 40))
 (segment (start 146.1262 136.398) (end 146.1262 126.753) (width 0.25) (layer "B.Cu") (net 41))
 (segment (start 148.6662 136.398) (end 148.6662 126.753) (width 0.25) (layer "B.Cu") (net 42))
 (segment (start 151.2062 136.398) (end 151.2062 126.753) (width 0.25) (layer "B.Cu") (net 43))
 (segment (start 153.7462 136.398) (end 153.7462 126.753) (width 0.25) (layer "B.Cu") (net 44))
 (segment (start 156.2862 136.398) (end 156.2862 126.753) (width 0.25) (layer "B.Cu") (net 45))
 (segment (start 158.8262 136.398) (end 158.8262 126.753) (width 0.25) (layer "B.Cu") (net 46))
 (segment (start 161.3662 136.398) (end 161.3662 126.753) (width 0.25) (layer "B.Cu") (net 47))
 (segment (start 163.9062 136.398) (end 163.9062 126.753) (width 0.25) (layer "B.Cu") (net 48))
 (segment (start 166.4462 136.398) (end 166.4462 126.753) (width 0.25) (layer "B.Cu") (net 49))
 (segment (start 168.9862 136.398) (end 168.9862 126.753) (width 0.25) (layer "B.Cu") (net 50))
 (segment (start 171.5262 136.398) (end 171.5262 126.753) (width 0.25) (layer "B.Cu") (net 51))
 (segment (start 174.0662 126.753) (end 174.0662 136.398) (width 0.25) (layer "B.Cu") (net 52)))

